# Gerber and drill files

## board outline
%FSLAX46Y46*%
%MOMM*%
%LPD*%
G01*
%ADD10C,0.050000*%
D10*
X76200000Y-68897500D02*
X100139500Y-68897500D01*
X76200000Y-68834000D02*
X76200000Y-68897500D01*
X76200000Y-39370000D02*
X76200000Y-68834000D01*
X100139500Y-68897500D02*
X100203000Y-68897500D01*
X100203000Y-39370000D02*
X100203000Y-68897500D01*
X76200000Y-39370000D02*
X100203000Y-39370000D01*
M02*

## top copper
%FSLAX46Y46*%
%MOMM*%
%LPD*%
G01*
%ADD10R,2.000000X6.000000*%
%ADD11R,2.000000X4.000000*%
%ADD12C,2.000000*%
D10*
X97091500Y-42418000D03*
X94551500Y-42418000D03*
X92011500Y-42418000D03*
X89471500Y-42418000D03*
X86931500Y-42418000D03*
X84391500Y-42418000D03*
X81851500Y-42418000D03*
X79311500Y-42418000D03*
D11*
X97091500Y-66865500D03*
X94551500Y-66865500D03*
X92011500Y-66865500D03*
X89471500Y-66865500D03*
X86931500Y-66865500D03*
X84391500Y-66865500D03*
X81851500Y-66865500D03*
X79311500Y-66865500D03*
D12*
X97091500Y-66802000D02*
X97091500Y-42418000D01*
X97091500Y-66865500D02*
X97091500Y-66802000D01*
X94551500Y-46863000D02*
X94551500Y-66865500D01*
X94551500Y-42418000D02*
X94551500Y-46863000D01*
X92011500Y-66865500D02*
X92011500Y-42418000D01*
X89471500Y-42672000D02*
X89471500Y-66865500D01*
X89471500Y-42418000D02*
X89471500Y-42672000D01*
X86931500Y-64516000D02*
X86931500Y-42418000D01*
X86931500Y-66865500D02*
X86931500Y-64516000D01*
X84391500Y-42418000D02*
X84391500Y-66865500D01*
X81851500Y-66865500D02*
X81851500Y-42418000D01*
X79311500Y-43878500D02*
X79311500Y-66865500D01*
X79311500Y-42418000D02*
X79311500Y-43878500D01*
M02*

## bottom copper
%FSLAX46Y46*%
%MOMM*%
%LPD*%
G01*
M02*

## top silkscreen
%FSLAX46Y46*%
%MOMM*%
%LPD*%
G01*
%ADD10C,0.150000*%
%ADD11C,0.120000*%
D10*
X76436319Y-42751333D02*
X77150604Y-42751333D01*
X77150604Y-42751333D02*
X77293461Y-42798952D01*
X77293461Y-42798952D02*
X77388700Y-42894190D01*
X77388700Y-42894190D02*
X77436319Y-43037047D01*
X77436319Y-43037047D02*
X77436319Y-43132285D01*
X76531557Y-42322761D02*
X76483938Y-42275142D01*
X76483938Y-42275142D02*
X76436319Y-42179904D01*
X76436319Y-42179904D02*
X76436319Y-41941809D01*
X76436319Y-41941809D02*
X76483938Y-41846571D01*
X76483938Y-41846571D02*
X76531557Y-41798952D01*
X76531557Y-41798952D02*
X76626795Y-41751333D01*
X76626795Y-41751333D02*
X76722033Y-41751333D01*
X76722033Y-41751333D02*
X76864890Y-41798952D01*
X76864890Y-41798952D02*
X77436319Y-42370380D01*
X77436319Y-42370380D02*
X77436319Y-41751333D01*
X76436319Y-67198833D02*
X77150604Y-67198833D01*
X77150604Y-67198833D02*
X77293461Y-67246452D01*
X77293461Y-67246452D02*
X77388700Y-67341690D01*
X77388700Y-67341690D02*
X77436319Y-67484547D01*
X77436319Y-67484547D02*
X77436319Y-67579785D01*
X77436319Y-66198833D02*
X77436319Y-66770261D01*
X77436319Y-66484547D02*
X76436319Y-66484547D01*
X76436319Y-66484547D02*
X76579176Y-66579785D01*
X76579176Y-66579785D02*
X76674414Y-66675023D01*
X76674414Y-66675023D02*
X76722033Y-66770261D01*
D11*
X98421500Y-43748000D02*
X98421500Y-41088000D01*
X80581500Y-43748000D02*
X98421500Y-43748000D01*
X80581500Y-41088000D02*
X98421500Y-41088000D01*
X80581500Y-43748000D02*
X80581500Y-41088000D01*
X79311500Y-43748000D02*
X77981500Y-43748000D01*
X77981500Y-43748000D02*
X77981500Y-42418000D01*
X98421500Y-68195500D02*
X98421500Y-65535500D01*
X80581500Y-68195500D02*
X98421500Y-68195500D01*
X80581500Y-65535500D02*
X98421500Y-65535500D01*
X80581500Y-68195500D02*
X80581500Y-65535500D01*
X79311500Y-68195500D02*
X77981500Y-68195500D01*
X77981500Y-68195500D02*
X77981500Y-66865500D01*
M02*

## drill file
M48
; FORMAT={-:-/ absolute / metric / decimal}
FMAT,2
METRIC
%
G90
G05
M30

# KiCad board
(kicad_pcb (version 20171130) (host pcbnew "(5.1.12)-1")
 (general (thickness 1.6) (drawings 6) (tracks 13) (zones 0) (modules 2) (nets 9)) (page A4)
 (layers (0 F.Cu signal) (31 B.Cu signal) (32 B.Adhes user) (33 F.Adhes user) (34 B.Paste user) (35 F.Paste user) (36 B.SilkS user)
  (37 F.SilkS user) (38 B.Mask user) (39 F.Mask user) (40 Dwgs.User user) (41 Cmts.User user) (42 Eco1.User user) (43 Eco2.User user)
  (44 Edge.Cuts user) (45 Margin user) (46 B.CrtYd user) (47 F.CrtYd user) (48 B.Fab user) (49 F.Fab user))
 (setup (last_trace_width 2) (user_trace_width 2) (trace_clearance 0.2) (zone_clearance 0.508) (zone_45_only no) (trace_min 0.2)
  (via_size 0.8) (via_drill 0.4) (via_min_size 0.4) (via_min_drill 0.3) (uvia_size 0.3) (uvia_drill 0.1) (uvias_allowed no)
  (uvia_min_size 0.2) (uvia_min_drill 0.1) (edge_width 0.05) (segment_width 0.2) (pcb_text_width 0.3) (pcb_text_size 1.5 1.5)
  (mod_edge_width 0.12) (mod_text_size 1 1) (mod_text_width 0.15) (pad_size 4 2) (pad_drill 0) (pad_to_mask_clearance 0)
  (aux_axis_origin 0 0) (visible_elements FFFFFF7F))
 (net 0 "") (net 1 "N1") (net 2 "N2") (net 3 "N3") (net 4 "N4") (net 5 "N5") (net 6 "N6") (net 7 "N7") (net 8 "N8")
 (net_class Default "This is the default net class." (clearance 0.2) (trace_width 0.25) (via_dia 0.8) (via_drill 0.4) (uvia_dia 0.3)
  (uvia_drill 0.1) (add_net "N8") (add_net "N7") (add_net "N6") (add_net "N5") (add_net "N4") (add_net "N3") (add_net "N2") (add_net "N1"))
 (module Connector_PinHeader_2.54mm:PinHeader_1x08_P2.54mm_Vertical (layer F.Cu) (at 79.3115 42.418 90)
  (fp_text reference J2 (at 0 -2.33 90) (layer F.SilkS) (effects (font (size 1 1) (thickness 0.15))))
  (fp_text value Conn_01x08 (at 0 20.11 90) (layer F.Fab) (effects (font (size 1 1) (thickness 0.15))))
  (fp_line (start -1.33 19.11) (end 1.33 19.11) (layer F.SilkS) (width 0.12))
  (fp_line (start -1.33 1.27) (end -1.33 19.11) (layer F.SilkS) (width 0.12))
  (fp_line (start 1.33 1.27) (end 1.33 19.11) (layer F.SilkS) (width 0.12))
  (fp_line (start -1.33 1.27) (end 1.33 1.27) (layer F.SilkS) (width 0.12))
  (fp_line (start -1.33 0) (end -1.33 -1.33) (layer F.SilkS) (width 0.12))
  (fp_line (start -1.33 -1.33) (end 0 -1.33) (layer F.SilkS) (width 0.12))
  (pad 8 smd rect (at 0 17.78 90) (size 6 2) (layers F.Cu F.Paste F.Mask) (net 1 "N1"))
  (pad 7 smd rect (at 0 15.24 90) (size 6 2) (layers F.Cu F.Paste F.Mask) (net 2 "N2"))
  (pad 6 smd rect (at 0 12.7 90) (size 6 2) (layers F.Cu F.Paste F.Mask) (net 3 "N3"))
  (pad 5 smd rect (at 0 10.16 90) (size 6 2) (layers F.Cu F.Paste F.Mask) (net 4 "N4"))
  (pad 4 smd rect (at 0 7.62 90) (size 6 2) (layers F.Cu F.Paste F.Mask) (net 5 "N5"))
  (pad 3 smd rect (at 0 5.08 90) (size 6 2) (layers F.Cu F.Paste F.Mask) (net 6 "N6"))
  (pad 2 smd rect (at 0 2.54 90) (size 6 2) (layers F.Cu F.Paste F.Mask) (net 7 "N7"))
  (pad 1 smd rect (at 0 0 90) (size 6 2) (layers F.Cu F.Paste F.Mask) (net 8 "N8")))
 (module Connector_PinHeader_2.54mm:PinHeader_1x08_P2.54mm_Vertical (layer F.Cu) (at 79.3115 66.8655 90)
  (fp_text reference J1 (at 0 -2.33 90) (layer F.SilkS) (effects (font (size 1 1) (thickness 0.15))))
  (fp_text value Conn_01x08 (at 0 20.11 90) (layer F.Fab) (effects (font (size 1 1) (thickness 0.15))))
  (fp_line (start -1.33 19.11) (end 1.33 19.11) (layer F.SilkS) (width 0.12))
  (fp_line (start -1.33 1.27) (end -1.33 19.11) (layer F.SilkS) (width 0.12))
  (fp_line (start 1.33 1.27) (end 1.33 19.11) (layer F.SilkS) (width 0.12))
  (fp_line (start -1.33 1.27) (end 1.33 1.27) (layer F.SilkS) (width 0.12))
  (fp_line (start -1.33 0) (end -1.33 -1.33) (layer F.SilkS) (width 0.12))
  (fp_line (start -1.33 -1.33) (end 0 -1.33) (layer F.SilkS) (width 0.12))
  (pad 8 smd rect (at 0 17.78 90) (size 4 2) (layers F.Cu F.Paste F.Mask) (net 1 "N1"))
  (pad 7 smd rect (at 0 15.24 90) (size 4 2) (layers F.Cu F.Paste F.Mask) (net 2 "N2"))
  (pad 6 smd rect (at 0 12.7 90) (size 4 2) (layers F.Cu F.Paste F.Mask) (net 3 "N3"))
  (pad 5 smd rect (at 0 10.16 90) (size 4 2) (layers F.Cu F.Paste F.Mask) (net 4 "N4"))
  (pad 4 smd rect (at 0 7.62 90) (size 4 2) (layers F.Cu F.Paste F.Mask) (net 5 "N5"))
  (pad 3 smd rect (at 0 5.08 90) (size 4 2) (layers F.Cu F.Paste F.Mask) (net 6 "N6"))
  (pad 2 smd rect (at 0 2.54 90) (size 4 2) (layers F.Cu F.Paste F.Mask) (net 7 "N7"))
  (pad 1 smd rect (at 0 0 90) (size 4 2) (layers F.Cu F.Paste F.Mask) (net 8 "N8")))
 (gr_line (start 76.2 68.8975) (end 100.1395 68.8975) (layer Edge.Cuts) (width 0.05))
 (gr_line (start 76.2 68.834) (end 76.2 68.8975) (layer Edge.Cuts) (width 0.05))
 (gr_line (start 76.2 39.37) (end 76.2 68.834) (layer Edge.Cuts) (width 0.05))
 (gr_line (start 100.1395 68.8975) (end 100.203 68.8975) (layer Edge.Cuts) (width 0.05))
 (gr_line (start 100.203 39.37) (end 100.203 68.8975) (layer Edge.Cuts) (width 0.05))
 (gr_line (start 76.2 39.37) (end 100.203 39.37) (layer Edge.Cuts) (width 0.05))
 (segment (start 97.0915 66.802) (end 97.0915 42.418) (width 2) (layer F.Cu) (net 1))
 (segment (start 97.0915 66.8655) (end 97.0915 66.802) (width 2) (layer F.Cu) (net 1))
 (segment (start 94.5515 46.863) (end 94.5515 66.8655) (width 2) (layer F.Cu) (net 2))
 (segment (start 94.5515 42.418) (end 94.5515 46.863) (width 2) (layer F.Cu) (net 2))
 (segment (start 92.0115 66.8655) (end 92.0115 42.418) (width 2) (layer F.Cu) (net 3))
 (segment (start 89.4715 42.672) (end 89.4715 66.8655) (width 2) (layer F.Cu) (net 4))
 (segment (start 89.4715 42.418) (end 89.4715 42.672) (width 2) (layer F.Cu) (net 4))
 (segment (start 86.9315 64.516) (end 86.9315 42.418) (width 2) (layer F.Cu) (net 5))
 (segment (start 86.9315 66.8655) (end 86.9315 64.516) (width 2) (layer F.Cu) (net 5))
 (segment (start 84.3915 42.418) (end 84.3915 66.8655) (width 2) (layer F.Cu) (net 6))
 (segment (start 81.8515 66.8655) (end 81.8515 42.418) (width 2) (layer F.Cu) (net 7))
 (segment (start 79.3115 43.8785) (end 79.3115 66.8655) (width 2) (layer F.Cu) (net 8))
 (segment (start 79.3115 42.418) (end 79.3115 43.8785) (width 2) (layer F.Cu) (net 8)))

